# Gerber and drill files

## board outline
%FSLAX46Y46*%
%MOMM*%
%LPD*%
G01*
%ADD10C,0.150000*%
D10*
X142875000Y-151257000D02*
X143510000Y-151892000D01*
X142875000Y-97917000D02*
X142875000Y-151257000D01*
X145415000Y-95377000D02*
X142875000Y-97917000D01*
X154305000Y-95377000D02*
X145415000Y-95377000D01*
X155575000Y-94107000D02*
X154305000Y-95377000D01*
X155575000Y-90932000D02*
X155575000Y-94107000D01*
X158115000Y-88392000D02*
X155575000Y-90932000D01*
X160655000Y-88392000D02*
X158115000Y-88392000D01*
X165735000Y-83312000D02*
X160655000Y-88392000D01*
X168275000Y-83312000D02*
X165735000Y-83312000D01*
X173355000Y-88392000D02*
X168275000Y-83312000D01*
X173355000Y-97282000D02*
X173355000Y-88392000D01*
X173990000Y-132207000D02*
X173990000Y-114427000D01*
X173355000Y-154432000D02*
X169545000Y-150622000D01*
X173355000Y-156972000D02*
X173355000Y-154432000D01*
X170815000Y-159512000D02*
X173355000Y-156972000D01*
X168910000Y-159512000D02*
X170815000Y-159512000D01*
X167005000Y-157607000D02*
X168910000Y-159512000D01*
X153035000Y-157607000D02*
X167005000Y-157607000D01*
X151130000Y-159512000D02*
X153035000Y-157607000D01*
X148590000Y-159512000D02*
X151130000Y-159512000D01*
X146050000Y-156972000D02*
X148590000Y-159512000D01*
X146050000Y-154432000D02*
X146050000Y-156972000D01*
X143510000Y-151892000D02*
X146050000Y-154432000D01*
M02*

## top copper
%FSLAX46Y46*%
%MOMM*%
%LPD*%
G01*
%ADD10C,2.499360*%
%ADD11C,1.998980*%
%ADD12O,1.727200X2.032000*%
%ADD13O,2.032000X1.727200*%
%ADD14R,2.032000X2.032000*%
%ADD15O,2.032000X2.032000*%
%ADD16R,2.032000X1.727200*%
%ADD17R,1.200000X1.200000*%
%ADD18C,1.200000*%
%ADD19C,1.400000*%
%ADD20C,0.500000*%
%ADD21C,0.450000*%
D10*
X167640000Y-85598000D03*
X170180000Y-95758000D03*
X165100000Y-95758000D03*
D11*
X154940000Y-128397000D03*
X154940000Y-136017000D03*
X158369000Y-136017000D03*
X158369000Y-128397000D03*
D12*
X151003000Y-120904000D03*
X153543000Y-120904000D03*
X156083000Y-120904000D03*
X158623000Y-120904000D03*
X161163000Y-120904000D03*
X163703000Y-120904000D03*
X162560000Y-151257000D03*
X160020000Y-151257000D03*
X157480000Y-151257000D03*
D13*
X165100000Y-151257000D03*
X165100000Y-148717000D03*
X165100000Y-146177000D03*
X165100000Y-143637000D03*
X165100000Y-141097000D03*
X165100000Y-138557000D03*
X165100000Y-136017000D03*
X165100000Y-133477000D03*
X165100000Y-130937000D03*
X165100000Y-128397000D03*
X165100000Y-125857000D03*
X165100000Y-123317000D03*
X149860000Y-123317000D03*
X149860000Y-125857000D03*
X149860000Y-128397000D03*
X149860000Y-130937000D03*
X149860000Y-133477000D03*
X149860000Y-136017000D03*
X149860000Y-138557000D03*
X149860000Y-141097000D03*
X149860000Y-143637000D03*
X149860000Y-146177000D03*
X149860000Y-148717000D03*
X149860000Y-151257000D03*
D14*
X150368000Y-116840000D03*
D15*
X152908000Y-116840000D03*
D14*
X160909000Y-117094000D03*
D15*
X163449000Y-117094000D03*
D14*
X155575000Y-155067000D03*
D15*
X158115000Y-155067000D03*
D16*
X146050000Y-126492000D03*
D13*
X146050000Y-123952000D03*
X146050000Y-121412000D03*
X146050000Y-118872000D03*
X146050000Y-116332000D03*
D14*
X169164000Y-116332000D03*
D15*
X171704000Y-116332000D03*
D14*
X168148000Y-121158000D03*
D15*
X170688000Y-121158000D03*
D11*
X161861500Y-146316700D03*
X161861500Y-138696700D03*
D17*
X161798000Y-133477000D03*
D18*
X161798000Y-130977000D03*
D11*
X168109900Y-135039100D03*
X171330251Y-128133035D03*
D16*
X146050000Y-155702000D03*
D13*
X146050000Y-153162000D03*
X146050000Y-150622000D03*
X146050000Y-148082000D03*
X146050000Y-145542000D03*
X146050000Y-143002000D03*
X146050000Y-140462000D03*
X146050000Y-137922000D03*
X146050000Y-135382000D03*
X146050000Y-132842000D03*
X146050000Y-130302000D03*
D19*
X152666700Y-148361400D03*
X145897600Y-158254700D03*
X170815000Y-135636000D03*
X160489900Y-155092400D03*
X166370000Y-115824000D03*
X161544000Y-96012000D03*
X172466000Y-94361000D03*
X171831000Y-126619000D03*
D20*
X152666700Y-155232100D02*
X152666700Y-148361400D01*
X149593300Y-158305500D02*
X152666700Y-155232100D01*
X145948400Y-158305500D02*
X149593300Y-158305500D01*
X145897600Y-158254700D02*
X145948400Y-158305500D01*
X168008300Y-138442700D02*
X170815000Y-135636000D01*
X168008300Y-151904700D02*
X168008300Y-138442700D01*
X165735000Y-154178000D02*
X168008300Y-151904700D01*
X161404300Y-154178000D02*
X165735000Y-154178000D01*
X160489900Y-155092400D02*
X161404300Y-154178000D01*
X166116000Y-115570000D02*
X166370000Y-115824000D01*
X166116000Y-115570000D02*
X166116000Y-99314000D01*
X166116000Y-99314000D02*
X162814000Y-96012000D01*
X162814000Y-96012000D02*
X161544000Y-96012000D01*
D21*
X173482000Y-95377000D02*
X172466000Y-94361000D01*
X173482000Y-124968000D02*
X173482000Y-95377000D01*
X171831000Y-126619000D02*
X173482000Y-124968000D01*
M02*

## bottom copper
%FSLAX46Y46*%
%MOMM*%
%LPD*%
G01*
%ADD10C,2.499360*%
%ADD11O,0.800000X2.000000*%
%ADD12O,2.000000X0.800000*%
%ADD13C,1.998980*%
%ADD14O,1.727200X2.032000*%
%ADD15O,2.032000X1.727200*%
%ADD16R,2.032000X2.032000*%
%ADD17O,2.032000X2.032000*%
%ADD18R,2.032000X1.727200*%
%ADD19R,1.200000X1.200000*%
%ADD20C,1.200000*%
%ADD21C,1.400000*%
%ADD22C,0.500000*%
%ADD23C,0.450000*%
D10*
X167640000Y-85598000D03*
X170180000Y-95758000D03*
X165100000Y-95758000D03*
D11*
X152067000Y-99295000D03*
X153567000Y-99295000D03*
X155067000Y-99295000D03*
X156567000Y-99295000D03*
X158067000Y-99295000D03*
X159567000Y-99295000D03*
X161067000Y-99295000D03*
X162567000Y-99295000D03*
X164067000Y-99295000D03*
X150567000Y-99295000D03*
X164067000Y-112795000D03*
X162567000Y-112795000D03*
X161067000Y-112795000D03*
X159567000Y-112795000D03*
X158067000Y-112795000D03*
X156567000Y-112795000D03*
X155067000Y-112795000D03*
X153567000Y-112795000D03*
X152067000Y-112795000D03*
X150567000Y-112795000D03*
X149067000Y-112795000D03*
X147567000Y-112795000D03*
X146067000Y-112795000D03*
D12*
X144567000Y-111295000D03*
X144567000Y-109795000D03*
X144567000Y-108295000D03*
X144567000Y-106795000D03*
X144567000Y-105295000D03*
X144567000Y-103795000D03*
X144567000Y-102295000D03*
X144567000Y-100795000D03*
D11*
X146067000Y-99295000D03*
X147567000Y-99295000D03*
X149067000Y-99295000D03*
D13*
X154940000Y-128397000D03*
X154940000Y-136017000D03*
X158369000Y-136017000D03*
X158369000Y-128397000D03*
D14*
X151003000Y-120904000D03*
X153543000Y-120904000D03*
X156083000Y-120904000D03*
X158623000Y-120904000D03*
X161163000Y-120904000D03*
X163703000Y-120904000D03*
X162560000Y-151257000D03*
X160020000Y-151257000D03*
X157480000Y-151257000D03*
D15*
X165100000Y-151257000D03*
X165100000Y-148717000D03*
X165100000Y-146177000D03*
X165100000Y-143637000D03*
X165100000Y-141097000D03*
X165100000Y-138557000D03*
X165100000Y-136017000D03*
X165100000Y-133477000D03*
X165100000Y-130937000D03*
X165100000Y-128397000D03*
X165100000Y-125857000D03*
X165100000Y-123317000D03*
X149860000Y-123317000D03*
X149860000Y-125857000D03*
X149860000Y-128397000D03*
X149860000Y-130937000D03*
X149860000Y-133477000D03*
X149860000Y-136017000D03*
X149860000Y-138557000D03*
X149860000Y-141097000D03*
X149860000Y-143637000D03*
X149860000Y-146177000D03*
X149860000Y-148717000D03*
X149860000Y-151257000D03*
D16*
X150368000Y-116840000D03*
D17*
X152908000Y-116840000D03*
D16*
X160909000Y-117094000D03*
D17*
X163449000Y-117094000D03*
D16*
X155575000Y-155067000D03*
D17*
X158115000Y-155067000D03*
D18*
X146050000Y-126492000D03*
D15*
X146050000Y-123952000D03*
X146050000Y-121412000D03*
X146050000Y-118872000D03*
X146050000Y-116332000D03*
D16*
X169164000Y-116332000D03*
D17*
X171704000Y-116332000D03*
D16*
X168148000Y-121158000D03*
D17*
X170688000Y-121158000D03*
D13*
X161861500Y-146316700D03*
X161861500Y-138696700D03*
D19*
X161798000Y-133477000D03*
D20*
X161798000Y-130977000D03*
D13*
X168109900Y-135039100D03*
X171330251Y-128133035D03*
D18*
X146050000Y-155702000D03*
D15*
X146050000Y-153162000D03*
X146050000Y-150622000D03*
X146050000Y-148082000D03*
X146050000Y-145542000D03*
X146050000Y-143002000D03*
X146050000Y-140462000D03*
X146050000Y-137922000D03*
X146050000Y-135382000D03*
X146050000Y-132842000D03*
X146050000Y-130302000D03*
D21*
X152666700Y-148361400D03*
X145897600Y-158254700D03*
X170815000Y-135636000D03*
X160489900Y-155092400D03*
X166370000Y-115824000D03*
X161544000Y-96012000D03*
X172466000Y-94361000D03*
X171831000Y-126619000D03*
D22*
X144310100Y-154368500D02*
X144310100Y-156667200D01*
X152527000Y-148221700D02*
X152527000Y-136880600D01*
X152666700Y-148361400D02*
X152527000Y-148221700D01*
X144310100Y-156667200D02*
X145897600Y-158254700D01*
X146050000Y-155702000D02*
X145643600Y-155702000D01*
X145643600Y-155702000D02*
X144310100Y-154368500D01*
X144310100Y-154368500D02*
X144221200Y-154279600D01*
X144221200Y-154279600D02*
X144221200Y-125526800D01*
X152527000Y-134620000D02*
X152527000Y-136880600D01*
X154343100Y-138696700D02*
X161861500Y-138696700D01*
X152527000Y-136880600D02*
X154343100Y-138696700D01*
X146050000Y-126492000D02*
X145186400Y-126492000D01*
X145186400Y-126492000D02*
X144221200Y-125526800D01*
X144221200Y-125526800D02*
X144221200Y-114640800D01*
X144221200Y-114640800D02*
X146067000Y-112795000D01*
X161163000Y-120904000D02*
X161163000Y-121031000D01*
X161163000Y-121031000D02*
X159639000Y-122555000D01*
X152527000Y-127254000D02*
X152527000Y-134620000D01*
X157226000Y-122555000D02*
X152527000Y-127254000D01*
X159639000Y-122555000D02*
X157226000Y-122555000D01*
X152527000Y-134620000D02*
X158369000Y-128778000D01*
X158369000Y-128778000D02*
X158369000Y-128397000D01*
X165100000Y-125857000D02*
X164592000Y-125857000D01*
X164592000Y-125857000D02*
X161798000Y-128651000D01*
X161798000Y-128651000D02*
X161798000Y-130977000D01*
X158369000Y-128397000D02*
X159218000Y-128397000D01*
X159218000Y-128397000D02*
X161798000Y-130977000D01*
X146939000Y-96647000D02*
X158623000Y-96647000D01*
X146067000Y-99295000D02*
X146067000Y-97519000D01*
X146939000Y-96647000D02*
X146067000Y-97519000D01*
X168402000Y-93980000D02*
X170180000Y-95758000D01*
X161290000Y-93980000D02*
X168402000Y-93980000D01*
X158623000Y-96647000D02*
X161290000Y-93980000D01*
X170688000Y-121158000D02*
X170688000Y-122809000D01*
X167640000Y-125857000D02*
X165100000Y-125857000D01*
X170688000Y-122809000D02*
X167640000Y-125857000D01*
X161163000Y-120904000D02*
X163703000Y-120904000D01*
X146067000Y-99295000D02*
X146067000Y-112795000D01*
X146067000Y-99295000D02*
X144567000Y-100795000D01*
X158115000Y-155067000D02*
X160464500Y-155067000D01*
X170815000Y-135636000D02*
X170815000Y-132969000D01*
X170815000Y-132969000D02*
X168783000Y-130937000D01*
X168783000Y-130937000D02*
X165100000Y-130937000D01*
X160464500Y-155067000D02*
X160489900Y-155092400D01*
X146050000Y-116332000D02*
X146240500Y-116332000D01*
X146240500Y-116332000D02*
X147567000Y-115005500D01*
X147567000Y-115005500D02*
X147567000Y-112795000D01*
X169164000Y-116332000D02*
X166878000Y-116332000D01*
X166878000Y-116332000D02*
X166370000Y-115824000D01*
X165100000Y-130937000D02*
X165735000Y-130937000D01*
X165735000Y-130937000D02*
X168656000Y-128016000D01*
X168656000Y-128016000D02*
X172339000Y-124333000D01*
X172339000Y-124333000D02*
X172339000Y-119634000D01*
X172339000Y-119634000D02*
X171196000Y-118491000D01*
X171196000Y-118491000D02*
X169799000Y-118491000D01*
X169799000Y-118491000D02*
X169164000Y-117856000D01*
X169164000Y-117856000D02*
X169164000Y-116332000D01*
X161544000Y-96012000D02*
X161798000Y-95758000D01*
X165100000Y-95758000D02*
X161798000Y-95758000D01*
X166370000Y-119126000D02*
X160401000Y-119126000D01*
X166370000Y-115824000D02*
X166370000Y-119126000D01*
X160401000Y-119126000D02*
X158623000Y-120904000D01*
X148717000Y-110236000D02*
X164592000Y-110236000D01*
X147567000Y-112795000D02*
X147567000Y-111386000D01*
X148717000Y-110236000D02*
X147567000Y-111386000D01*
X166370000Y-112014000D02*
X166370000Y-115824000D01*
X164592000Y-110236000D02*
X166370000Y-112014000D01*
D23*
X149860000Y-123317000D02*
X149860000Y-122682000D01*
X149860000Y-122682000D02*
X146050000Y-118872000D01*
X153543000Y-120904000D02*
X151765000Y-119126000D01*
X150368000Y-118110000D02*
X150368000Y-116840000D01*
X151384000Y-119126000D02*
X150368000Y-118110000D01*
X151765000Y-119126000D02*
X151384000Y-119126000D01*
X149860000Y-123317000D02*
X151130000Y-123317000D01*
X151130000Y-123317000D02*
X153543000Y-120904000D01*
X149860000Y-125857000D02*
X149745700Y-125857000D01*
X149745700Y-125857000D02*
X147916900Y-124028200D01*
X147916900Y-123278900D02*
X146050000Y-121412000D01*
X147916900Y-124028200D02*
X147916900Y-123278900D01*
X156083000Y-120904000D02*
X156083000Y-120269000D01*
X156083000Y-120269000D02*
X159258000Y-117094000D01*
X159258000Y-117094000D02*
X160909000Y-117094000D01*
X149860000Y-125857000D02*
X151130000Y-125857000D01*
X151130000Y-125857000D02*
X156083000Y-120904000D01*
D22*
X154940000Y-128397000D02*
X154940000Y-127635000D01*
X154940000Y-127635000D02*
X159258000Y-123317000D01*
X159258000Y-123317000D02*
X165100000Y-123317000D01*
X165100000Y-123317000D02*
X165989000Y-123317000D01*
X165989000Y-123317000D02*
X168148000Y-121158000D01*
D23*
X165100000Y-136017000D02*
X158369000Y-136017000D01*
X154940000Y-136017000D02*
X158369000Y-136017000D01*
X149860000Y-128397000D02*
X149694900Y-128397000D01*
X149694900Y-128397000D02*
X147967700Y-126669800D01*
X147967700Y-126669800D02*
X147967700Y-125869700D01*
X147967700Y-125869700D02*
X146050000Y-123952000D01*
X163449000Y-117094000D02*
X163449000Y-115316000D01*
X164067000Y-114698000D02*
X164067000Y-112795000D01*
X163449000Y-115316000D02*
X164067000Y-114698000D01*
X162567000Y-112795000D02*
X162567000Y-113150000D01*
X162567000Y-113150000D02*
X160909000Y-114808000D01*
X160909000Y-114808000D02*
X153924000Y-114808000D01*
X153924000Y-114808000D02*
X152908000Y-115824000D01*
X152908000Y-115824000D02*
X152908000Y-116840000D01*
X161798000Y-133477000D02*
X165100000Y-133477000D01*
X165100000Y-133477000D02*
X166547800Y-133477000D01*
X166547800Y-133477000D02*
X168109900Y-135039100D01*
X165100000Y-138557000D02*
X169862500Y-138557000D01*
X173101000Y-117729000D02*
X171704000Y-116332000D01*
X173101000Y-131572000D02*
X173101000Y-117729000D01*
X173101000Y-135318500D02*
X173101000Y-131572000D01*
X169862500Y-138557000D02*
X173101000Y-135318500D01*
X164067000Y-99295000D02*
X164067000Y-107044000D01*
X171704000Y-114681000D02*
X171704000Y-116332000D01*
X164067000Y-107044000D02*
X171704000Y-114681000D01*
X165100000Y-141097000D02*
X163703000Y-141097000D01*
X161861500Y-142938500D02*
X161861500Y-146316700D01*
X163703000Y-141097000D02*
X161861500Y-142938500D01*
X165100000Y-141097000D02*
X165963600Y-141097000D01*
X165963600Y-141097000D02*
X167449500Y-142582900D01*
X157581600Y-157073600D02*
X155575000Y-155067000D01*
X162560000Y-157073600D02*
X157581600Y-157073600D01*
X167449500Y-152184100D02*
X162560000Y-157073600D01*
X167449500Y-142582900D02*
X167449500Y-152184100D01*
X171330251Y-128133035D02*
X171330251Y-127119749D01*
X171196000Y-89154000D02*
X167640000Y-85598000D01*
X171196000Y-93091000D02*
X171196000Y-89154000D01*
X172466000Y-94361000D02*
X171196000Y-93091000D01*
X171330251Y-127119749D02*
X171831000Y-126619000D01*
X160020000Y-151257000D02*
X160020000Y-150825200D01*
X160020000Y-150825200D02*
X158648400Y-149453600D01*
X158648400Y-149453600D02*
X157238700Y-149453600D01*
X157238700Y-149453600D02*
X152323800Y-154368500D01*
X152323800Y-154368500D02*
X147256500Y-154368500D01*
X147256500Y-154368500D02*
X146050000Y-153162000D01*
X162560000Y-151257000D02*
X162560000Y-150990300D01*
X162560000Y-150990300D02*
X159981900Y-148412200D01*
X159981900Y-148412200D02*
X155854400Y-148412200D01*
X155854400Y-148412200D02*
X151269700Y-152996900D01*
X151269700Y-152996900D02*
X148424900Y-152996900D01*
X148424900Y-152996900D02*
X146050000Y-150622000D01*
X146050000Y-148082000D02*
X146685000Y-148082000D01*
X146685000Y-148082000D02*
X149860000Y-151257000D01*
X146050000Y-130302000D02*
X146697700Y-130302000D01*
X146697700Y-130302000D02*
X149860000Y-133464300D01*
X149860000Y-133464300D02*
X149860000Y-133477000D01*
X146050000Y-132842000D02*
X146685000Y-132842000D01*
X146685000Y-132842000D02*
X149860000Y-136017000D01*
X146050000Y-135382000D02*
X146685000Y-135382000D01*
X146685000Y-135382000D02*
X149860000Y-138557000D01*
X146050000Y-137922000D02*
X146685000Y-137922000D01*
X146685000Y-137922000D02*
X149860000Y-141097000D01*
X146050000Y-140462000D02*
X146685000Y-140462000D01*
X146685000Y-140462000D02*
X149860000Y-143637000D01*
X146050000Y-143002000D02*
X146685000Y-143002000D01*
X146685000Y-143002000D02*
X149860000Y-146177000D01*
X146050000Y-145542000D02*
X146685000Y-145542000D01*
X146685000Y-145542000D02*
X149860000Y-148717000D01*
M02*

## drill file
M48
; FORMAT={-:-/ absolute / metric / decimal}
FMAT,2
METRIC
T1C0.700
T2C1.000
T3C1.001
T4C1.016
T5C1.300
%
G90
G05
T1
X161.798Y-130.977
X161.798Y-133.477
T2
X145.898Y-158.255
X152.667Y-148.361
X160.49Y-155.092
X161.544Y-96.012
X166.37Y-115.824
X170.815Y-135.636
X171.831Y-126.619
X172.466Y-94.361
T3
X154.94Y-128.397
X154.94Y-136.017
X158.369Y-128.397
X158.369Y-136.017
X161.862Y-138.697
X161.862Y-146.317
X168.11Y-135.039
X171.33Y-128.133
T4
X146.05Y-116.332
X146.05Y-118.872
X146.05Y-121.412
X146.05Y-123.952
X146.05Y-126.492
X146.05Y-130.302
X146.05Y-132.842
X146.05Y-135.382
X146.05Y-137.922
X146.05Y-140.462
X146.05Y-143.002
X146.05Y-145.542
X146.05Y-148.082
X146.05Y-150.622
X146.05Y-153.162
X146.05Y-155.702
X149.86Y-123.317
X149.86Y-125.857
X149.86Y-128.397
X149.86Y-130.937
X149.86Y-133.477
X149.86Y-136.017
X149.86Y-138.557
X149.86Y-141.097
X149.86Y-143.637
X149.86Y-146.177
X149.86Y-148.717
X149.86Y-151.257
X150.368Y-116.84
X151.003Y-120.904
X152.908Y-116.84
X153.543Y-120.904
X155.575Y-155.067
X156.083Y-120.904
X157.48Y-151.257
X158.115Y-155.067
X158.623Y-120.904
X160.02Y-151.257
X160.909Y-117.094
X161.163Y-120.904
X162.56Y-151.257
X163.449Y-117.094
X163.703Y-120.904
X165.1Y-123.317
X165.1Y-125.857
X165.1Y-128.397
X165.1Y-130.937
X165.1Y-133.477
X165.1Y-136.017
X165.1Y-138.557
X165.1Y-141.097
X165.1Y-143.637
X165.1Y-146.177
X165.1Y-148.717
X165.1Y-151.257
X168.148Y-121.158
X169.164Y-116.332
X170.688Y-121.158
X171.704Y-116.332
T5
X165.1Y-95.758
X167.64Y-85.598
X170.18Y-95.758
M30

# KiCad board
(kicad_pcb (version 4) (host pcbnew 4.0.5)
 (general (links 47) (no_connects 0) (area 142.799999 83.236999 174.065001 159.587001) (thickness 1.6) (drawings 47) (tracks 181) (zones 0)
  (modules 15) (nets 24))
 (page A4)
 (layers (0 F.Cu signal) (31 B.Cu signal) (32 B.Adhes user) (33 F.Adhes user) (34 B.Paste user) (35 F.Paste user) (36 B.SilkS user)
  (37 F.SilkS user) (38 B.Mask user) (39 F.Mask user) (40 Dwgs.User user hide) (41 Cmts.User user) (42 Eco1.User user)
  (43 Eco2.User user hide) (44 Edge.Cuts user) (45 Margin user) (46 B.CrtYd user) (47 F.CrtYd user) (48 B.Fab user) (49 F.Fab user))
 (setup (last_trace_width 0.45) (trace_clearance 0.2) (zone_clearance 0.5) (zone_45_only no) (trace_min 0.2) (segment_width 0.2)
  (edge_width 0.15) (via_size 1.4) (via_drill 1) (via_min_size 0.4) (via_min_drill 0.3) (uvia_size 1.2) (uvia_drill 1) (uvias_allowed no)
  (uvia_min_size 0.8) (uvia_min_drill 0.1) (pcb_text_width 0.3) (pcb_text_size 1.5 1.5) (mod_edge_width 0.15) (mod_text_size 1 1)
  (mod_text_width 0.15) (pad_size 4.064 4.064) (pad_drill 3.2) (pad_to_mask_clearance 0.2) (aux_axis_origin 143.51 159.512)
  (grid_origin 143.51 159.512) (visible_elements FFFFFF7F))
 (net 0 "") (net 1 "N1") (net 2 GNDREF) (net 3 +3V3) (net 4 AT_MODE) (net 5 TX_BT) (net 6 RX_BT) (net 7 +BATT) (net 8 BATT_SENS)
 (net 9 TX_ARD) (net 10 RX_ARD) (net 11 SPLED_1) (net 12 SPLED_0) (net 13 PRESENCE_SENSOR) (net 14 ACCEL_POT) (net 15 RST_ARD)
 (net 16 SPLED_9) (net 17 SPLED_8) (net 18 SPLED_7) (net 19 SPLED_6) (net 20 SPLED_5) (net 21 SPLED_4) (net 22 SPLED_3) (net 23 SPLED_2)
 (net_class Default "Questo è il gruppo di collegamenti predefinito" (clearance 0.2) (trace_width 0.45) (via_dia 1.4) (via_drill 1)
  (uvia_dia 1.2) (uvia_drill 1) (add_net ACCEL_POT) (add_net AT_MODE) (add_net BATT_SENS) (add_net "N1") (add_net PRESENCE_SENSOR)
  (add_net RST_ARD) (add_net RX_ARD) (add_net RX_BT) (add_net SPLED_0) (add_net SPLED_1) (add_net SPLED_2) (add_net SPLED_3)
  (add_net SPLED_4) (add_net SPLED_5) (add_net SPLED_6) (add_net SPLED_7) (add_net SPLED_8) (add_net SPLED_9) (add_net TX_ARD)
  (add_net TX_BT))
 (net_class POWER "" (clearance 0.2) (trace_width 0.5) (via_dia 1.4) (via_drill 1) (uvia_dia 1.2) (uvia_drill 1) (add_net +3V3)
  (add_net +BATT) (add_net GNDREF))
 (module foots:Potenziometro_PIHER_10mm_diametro (layer F.Cu) (at 165.1 95.758)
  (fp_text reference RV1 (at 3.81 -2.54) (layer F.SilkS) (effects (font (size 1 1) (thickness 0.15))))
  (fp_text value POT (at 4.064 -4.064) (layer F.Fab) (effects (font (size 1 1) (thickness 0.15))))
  (pad 2 thru_hole circle (at 2.54 -10.16) (size 2.49936 2.49936) (drill 1.30048) (layers *.Cu *.Mask) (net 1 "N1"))
  (pad 3 thru_hole circle (at 5.08 0) (size 2.49936 2.49936) (drill 1.30048) (layers *.Cu *.Mask) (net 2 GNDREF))
  (pad 1 thru_hole circle (at 0 0) (size 2.49936 2.49936) (drill 1.30048) (layers *.Cu *.Mask) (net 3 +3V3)))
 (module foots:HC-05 (layer B.Cu) (at 155.067 106.045 90)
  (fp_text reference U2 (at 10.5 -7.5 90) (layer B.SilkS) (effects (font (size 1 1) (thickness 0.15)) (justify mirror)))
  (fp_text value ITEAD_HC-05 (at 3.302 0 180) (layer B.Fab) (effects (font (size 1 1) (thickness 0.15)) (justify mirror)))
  (pad 26 smd oval (at 6.75 -3 90) (size 2 0.8) (layers B.Cu B.Paste B.Mask))
  (pad 27 smd oval (at 6.75 -1.5 90) (size 2 0.8) (layers B.Cu B.Paste B.Mask))
  (pad 28 smd oval (at 6.75 0 90) (size 2 0.8) (layers B.Cu B.Paste B.Mask))
  (pad 29 smd oval (at 6.75 1.5 90) (size 2 0.8) (layers B.Cu B.Paste B.Mask))
  (pad 30 smd oval (at 6.75 3 90) (size 2 0.8) (layers B.Cu B.Paste B.Mask))
  (pad 31 smd oval (at 6.75 4.5 90) (size 2 0.8) (layers B.Cu B.Paste B.Mask))
  (pad 32 smd oval (at 6.75 6 90) (size 2 0.8) (layers B.Cu B.Paste B.Mask))
  (pad 33 smd oval (at 6.75 7.5 90) (size 2 0.8) (layers B.Cu B.Paste B.Mask))
  (pad 34 smd oval (at 6.75 9 90) (size 2 0.8) (layers B.Cu B.Paste B.Mask) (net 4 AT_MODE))
  (pad 25 smd oval (at 6.75 -4.5 90) (size 2 0.8) (layers B.Cu B.Paste B.Mask))
  (pad 1 smd oval (at -6.75 9 90) (size 2 0.8) (layers B.Cu B.Paste B.Mask) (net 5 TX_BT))
  (pad 2 smd oval (at -6.75 7.5 90) (size 2 0.8) (layers B.Cu B.Paste B.Mask) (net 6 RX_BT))
  (pad 3 smd oval (at -6.75 6 90) (size 2 0.8) (layers B.Cu B.Paste B.Mask))
  (pad 4 smd oval (at -6.75 4.5 90) (size 2 0.8) (layers B.Cu B.Paste B.Mask))
  (pad 5 smd oval (at -6.75 3 90) (size 2 0.8) (layers B.Cu B.Paste B.Mask))
  (pad 6 smd oval (at -6.75 1.5 90) (size 2 0.8) (layers B.Cu B.Paste B.Mask))
  (pad 7 smd oval (at -6.75 0 90) (size 2 0.8) (layers B.Cu B.Paste B.Mask))
  (pad 8 smd oval (at -6.75 -1.5 90) (size 2 0.8) (layers B.Cu B.Paste B.Mask))
  (pad 9 smd oval (at -6.75 -3 90) (size 2 0.8) (layers B.Cu B.Paste B.Mask))
  (pad 10 smd oval (at -6.75 -4.5 90) (size 2 0.8) (layers B.Cu B.Paste B.Mask))
  (pad 11 smd oval (at -6.75 -6 90) (size 2 0.8) (layers B.Cu B.Paste B.Mask))
  (pad 12 smd oval (at -6.75 -7.5 90) (size 2 0.8) (layers B.Cu B.Paste B.Mask) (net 3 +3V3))
  (pad 13 smd oval (at -6.75 -9 90) (size 2 0.8) (layers B.Cu B.Paste B.Mask) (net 2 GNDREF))
  (pad 14 smd oval (at -5.25 -10.5) (size 2 0.8) (layers B.Cu B.Paste B.Mask))
  (pad 15 smd oval (at -3.75 -10.5 180) (size 2 0.8) (layers B.Cu B.Paste B.Mask))
  (pad 16 smd oval (at -2.25 -10.5 180) (size 2 0.8) (layers B.Cu B.Paste B.Mask))
  (pad 17 smd oval (at -0.75 -10.5 180) (size 2 0.8) (layers B.Cu B.Paste B.Mask))
  (pad 18 smd oval (at 0.75 -10.5 180) (size 2 0.8) (layers B.Cu B.Paste B.Mask))
  (pad 19 smd oval (at 2.25 -10.5 180) (size 2 0.8) (layers B.Cu B.Paste B.Mask))
  (pad 20 smd oval (at 3.75 -10.5 180) (size 2 0.8) (layers B.Cu B.Paste B.Mask))
  (pad 21 smd oval (at 5.25 -10.5 180) (size 2 0.8) (layers B.Cu B.Paste B.Mask) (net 2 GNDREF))
  (pad 22 smd oval (at 6.75 -9 90) (size 2 0.8) (layers B.Cu B.Paste B.Mask) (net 2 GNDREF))
  (pad 23 smd oval (at 6.75 -7.5 90) (size 2 0.8) (layers B.Cu B.Paste B.Mask))
  (pad 24 smd oval (at 6.75 -6 90) (size 2 0.8) (layers B.Cu B.Paste B.Mask)))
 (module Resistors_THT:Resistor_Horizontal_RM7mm (layer F.Cu) (at 154.94 128.397 270)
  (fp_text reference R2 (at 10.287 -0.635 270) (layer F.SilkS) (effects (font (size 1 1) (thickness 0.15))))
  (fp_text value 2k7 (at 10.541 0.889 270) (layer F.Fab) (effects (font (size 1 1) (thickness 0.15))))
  (pad 1 thru_hole circle (at 0 0 270) (size 1.99898 1.99898) (drill 1.00076) (layers *.Cu *.SilkS *.Mask) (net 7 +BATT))
  (pad 2 thru_hole circle (at 7.62 0 270) (size 1.99898 1.99898) (drill 1.00076) (layers *.Cu *.SilkS *.Mask) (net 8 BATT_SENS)))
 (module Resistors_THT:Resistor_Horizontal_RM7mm (layer F.Cu) (at 158.369 136.017 90)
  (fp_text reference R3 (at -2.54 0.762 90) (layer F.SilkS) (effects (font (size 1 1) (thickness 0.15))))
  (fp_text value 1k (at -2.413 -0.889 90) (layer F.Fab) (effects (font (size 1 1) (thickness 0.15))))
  (pad 1 thru_hole circle (at 0 0 90) (size 1.99898 1.99898) (drill 1.00076) (layers *.Cu *.SilkS *.Mask) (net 8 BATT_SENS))
  (pad 2 thru_hole circle (at 7.62 0 90) (size 1.99898 1.99898) (drill 1.00076) (layers *.Cu *.SilkS *.Mask)))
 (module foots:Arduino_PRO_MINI (layer F.Cu) (at 157.48 120.777)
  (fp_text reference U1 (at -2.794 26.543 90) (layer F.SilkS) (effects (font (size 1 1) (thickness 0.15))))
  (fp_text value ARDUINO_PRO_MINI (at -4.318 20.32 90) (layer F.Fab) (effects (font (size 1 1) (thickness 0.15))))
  (pad 33 thru_hole oval (at -6.477 0.127 90) (size 2.032 1.7272) (drill 1.016) (layers *.Cu *.Mask))
  (pad 32 thru_hole oval (at -3.937 0.127 90) (size 2.032 1.7272) (drill 1.016) (layers *.Cu *.Mask) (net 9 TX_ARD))
  (pad 31 thru_hole oval (at -1.397 0.127 90) (size 2.032 1.7272) (drill 1.016) (layers *.Cu *.Mask) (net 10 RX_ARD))
  (pad 30 thru_hole oval (at 1.143 0.127 90) (size 2.032 1.7272) (drill 1.016) (layers *.Cu *.Mask) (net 3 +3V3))
  (pad 29 thru_hole oval (at 3.683 0.127 90) (size 2.032 1.7272) (drill 1.016) (layers *.Cu *.Mask) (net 2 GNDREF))
  (pad 28 thru_hole oval (at 6.223 0.127 90) (size 2.032 1.7272) (drill 1.016) (layers *.Cu *.Mask) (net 2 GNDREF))
  (pad 15 thru_hole oval (at 5.08 30.48 90) (size 2.032 1.7272) (drill 1.016) (layers *.Cu *.Mask) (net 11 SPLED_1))
  (pad 14 thru_hole oval (at 2.54 30.48 90) (size 2.032 1.7272) (drill 1.016) (layers *.Cu *.Mask) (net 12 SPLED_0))
  (pad 13 thru_hole oval (at 0 30.48 90) (size 2.032 1.7272) (drill 1.016) (layers *.Cu *.Mask))
  (pad 16 thru_hole oval (at 7.62 30.48) (size 2.032 1.7272) (drill 1.016) (layers *.Cu *.Mask))
  (pad 17 thru_hole oval (at 7.62 27.94) (size 2.032 1.7272) (drill 1.016) (layers *.Cu *.Mask))
  (pad 18 thru_hole oval (at 7.62 25.4) (size 2.032 1.7272) (drill 1.016) (layers *.Cu *.Mask))
  (pad 19 thru_hole oval (at 7.62 22.86) (size 2.032 1.7272) (drill 1.016) (layers *.Cu *.Mask))
  (pad 20 thru_hole oval (at 7.62 20.32) (size 2.032 1.7272) (drill 1.016) (layers *.Cu *.Mask) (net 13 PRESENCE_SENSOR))
  (pad 21 thru_hole oval (at 7.62 17.78) (size 2.032 1.7272) (drill 1.016) (layers *.Cu *.Mask) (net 4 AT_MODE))
  (pad 22 thru_hole oval (at 7.62 15.24) (size 2.032 1.7272) (drill 1.016) (layers *.Cu *.Mask) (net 8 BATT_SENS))
  (pad 23 thru_hole oval (at 7.62 12.7) (size 2.032 1.7272) (drill 1.016) (layers *.Cu *.Mask) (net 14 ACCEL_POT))
  (pad 24 thru_hole oval (at 7.62 10.16) (size 2.032 1.7272) (drill 1.016) (layers *.Cu *.Mask) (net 3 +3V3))
  (pad 25 thru_hole oval (at 7.62 7.62) (size 2.032 1.7272) (drill 1.016) (layers *.Cu *.Mask))
  (pad 26 thru_hole oval (at 7.62 5.08) (size 2.032 1.7272) (drill 1.016) (layers *.Cu *.Mask) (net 2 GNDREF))
  (pad 27 thru_hole oval (at 7.62 2.54) (size 2.032 1.7272) (drill 1.016) (layers *.Cu *.Mask) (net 7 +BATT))
  (pad 1 thru_hole oval (at -7.62 2.54) (size 2.032 1.7272) (drill 1.016) (layers *.Cu *.Mask) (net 9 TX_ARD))
  (pad 2 thru_hole oval (at -7.62 5.08) (size 2.032 1.7272) (drill 1.016) (layers *.Cu *.Mask) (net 10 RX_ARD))
  (pad 3 thru_hole oval (at -7.62 7.62) (size 2.032 1.7272) (drill 1.016) (layers *.Cu *.Mask) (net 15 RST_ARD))
  (pad 4 thru_hole oval (at -7.62 10.16) (size 2.032 1.7272) (drill 1.016) (layers *.Cu *.Mask))
  (pad 5 thru_hole oval (at -7.62 12.7) (size 2.032 1.7272) (drill 1.016) (layers *.Cu *.Mask) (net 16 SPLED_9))
  (pad 6 thru_hole oval (at -7.62 15.24) (size 2.032 1.7272) (drill 1.016) (layers *.Cu *.Mask) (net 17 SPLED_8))
  (pad 7 thru_hole oval (at -7.62 17.78) (size 2.032 1.7272) (drill 1.016) (layers *.Cu *.Mask) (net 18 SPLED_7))
  (pad 8 thru_hole oval (at -7.62 20.32) (size 2.032 1.7272) (drill 1.016) (layers *.Cu *.Mask) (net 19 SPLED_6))
  (pad 9 thru_hole oval (at -7.62 22.86) (size 2.032 1.7272) (drill 1.016) (layers *.Cu *.Mask) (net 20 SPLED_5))
  (pad 10 thru_hole oval (at -7.62 25.4) (size 2.032 1.7272) (drill 1.016) (layers *.Cu *.Mask) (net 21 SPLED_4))
  (pad 11 thru_hole oval (at -7.62 27.94) (size 2.032 1.7272) (drill 1.016) (layers *.Cu *.Mask) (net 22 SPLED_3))
  (pad 12 thru_hole oval (at -7.62 30.48) (size 2.032 1.7272) (drill 1.016) (layers *.Cu *.Mask) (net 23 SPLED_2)))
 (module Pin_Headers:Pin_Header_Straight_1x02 (layer F.Cu) (at 150.368 116.84 90)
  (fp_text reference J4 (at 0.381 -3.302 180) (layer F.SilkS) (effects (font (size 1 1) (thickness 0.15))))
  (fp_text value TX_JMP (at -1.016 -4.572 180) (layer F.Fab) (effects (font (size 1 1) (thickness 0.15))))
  (pad 1 thru_hole rect (at 0 0 90) (size 2.032 2.032) (drill 1.016) (layers *.Cu *.Mask) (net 9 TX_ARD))
  (pad 2 thru_hole oval (at 0 2.54 90) (size 2.032 2.032) (drill 1.016) (layers *.Cu *.Mask) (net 6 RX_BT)))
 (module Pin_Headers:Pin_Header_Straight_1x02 (layer F.Cu) (at 160.909 117.094 90)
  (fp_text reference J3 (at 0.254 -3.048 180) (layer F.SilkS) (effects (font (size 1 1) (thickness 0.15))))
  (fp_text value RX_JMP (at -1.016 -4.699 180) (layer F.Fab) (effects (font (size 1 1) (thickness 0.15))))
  (pad 1 thru_hole rect (at 0 0 90) (size 2.032 2.032) (drill 1.016) (layers *.Cu *.Mask) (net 10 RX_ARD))
  (pad 2 thru_hole oval (at 0 2.54 90) (size 2.032 2.032) (drill 1.016) (layers *.Cu *.Mask) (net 5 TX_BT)))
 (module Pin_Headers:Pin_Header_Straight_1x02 (layer F.Cu) (at 155.575 155.067 90)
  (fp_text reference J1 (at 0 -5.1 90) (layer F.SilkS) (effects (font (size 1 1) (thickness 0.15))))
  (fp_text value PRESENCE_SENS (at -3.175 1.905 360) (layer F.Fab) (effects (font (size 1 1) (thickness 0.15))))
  (pad 1 thru_hole rect (at 0 0 90) (size 2.032 2.032) (drill 1.016) (layers *.Cu *.Mask) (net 13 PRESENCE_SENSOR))
  (pad 2 thru_hole oval (at 0 2.54 90) (size 2.032 2.032) (drill 1.016) (layers *.Cu *.Mask) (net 3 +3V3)))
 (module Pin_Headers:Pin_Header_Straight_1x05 (layer F.Cu) (at 146.05 126.492 180)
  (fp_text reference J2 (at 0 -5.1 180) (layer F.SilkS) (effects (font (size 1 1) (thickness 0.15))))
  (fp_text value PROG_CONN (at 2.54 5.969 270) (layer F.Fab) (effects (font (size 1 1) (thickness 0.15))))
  (pad 1 thru_hole rect (at 0 0 180) (size 2.032 1.7272) (drill 1.016) (layers *.Cu *.Mask) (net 2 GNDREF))
  (pad 2 thru_hole oval (at 0 2.54 180) (size 2.032 1.7272) (drill 1.016) (layers *.Cu *.Mask) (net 15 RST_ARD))
  (pad 3 thru_hole oval (at 0 5.08 180) (size 2.032 1.7272) (drill 1.016) (layers *.Cu *.Mask) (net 10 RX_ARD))
  (pad 4 thru_hole oval (at 0 7.62 180) (size 2.032 1.7272) (drill 1.016) (layers *.Cu *.Mask) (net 9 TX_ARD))
  (pad 5 thru_hole oval (at 0 10.16 180) (size 2.032 1.7272) (drill 1.016) (layers *.Cu *.Mask) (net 3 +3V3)))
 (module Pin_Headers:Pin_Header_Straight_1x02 (layer F.Cu) (at 169.164 116.332 90)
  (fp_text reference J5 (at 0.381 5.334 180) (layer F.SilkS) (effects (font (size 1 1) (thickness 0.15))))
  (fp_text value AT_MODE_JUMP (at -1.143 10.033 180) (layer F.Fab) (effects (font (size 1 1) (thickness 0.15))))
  (pad 1 thru_hole rect (at 0 0 90) (size 2.032 2.032) (drill 1.016) (layers *.Cu *.Mask) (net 3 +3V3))
  (pad 2 thru_hole oval (at 0 2.54 90) (size 2.032 2.032) (drill 1.016) (layers *.Cu *.Mask) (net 4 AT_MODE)))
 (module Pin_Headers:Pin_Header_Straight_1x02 (layer F.Cu) (at 168.148 121.158 90)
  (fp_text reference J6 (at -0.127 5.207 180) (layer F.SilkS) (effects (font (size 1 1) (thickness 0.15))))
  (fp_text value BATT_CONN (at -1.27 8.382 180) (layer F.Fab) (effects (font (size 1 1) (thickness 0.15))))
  (pad 1 thru_hole rect (at 0 0 90) (size 2.032 2.032) (drill 1.016) (layers *.Cu *.Mask) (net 7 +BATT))
  (pad 2 thru_hole oval (at 0 2.54 90) (size 2.032 2.032) (drill 1.016) (layers *.Cu *.Mask) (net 2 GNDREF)))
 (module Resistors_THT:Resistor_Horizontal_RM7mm (layer F.Cu) (at 161.8615 146.3167 90)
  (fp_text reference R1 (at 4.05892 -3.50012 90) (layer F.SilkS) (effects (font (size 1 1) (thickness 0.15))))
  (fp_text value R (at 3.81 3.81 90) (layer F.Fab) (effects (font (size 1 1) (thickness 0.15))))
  (pad 1 thru_hole circle (at 0 0 90) (size 1.99898 1.99898) (drill 1.00076) (layers *.Cu *.SilkS *.Mask) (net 13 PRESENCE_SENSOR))
  (pad 2 thru_hole circle (at 7.62 0 90) (size 1.99898 1.99898) (drill 1.00076) (layers *.Cu *.SilkS *.Mask) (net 2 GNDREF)))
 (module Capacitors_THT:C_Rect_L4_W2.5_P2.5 (layer F.Cu) (at 161.798 133.477 90)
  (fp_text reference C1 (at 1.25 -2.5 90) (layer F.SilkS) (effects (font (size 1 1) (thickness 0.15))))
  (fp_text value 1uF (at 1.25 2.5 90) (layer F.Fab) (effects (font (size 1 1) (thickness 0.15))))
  (pad 1 thru_hole rect (at 0 0 90) (size 1.2 1.2) (drill 0.7) (layers *.Cu *.Mask) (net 14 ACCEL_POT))
  (pad 2 thru_hole circle (at 2.5 0 90) (size 1.2 1.2) (drill 0.7) (layers *.Cu *.Mask) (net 2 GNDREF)))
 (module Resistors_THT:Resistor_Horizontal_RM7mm (layer F.Cu) (at 168.1099 135.0391 65)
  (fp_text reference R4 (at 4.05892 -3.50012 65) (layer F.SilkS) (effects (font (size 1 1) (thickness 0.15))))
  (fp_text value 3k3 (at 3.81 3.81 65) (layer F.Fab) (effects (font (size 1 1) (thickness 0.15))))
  (pad 1 thru_hole circle (at 0 0 65) (size 1.99898 1.99898) (drill 1.00076) (layers *.Cu *.SilkS *.Mask) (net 14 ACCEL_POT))
  (pad 2 thru_hole circle (at 7.62 0 65) (size 1.99898 1.99898) (drill 1.00076) (layers *.Cu *.SilkS *.Mask) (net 1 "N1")))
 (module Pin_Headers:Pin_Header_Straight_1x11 (layer F.Cu) (at 146.05 155.702 180)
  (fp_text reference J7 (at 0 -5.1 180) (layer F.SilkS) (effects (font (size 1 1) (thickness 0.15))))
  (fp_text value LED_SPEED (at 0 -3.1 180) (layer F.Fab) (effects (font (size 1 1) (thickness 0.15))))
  (pad 1 thru_hole rect (at 0 0 180) (size 2.032 1.7272) (drill 1.016) (layers *.Cu *.Mask) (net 2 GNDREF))
  (pad 2 thru_hole oval (at 0 2.54 180) (size 2.032 1.7272) (drill 1.016) (layers *.Cu *.Mask) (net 12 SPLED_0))
  (pad 3 thru_hole oval (at 0 5.08 180) (size 2.032 1.7272) (drill 1.016) (layers *.Cu *.Mask) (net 11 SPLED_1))
  (pad 4 thru_hole oval (at 0 7.62 180) (size 2.032 1.7272) (drill 1.016) (layers *.Cu *.Mask) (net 23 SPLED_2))
  (pad 5 thru_hole oval (at 0 10.16 180) (size 2.032 1.7272) (drill 1.016) (layers *.Cu *.Mask) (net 22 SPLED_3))
  (pad 6 thru_hole oval (at 0 12.7 180) (size 2.032 1.7272) (drill 1.016) (layers *.Cu *.Mask) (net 21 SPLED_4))
  (pad 7 thru_hole oval (at 0 15.24 180) (size 2.032 1.7272) (drill 1.016) (layers *.Cu *.Mask) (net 20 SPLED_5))
  (pad 8 thru_hole oval (at 0 17.78 180) (size 2.032 1.7272) (drill 1.016) (layers *.Cu *.Mask) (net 19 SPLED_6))
  (pad 9 thru_hole oval (at 0 20.32 180) (size 2.032 1.7272) (drill 1.016) (layers *.Cu *.Mask) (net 18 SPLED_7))
  (pad 10 thru_hole oval (at 0 22.86 180) (size 2.032 1.7272) (drill 1.016) (layers *.Cu *.Mask) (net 17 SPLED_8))
  (pad 11 thru_hole oval (at 0 25.4 180) (size 2.032 1.7272) (drill 1.016) (layers *.Cu *.Mask) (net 16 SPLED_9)))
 (gr_line (start 142.875 151.257) (end 143.51 151.892) (angle 90) (layer Edge.Cuts) (width 0.15))
 (gr_line (start 142.875 97.917) (end 142.875 151.257) (angle 90) (layer Edge.Cuts) (width 0.15))
 (gr_line (start 145.415 95.377) (end 142.875 97.917) (angle 90) (layer Edge.Cuts) (width 0.15))
 (gr_line (start 154.305 95.377) (end 145.415 95.377) (angle 90) (layer Edge.Cuts) (width 0.15))
 (gr_line (start 155.575 94.107) (end 154.305 95.377) (angle 90) (layer Edge.Cuts) (width 0.15))
 (gr_line (start 155.575 90.932) (end 155.575 94.107) (angle 90) (layer Edge.Cuts) (width 0.15))
 (gr_line (start 158.115 88.392) (end 155.575 90.932) (angle 90) (layer Edge.Cuts) (width 0.15))
 (gr_line (start 160.655 88.392) (end 158.115 88.392) (angle 90) (layer Edge.Cuts) (width 0.15))
 (gr_line (start 165.735 83.312) (end 160.655 88.392) (angle 90) (layer Edge.Cuts) (width 0.15))
 (gr_line (start 168.275 83.312) (end 165.735 83.312) (angle 90) (layer Edge.Cuts) (width 0.15))
 (gr_line (start 173.355 88.392) (end 168.275 83.312) (angle 90) (layer Edge.Cuts) (width 0.15))
 (gr_line (start 173.355 97.282) (end 173.355 88.392) (angle 90) (layer Edge.Cuts) (width 0.15))
 (gr_line (start 173.99 132.207) (end 173.99 114.427) (angle 90) (layer Edge.Cuts) (width 0.15))
 (gr_line (start 173.355 154.432) (end 169.545 150.622) (angle 90) (layer Edge.Cuts) (width 0.15))
 (gr_line (start 173.355 156.972) (end 173.355 154.432) (angle 90) (layer Edge.Cuts) (width 0.15))
 (gr_line (start 170.815 159.512) (end 173.355 156.972) (angle 90) (layer Edge.Cuts) (width 0.15))
 (gr_line (start 168.91 159.512) (end 170.815 159.512) (angle 90) (layer Edge.Cuts) (width 0.15))
 (gr_line (start 167.005 157.607) (end 168.91 159.512) (angle 90) (layer Edge.Cuts) (width 0.15))
 (gr_line (start 153.035 157.607) (end 167.005 157.607) (angle 90) (layer Edge.Cuts) (width 0.15))
 (gr_line (start 151.13 159.512) (end 153.035 157.607) (angle 90) (layer Edge.Cuts) (width 0.15))
 (gr_line (start 148.59 159.512) (end 151.13 159.512) (angle 90) (layer Edge.Cuts) (width 0.15))
 (gr_line (start 146.05 156.972) (end 148.59 159.512) (angle 90) (layer Edge.Cuts) (width 0.15))
 (gr_line (start 146.05 154.432) (end 146.05 156.972) (angle 90) (layer Edge.Cuts) (width 0.15))
 (gr_line (start 143.51 151.892) (end 146.05 154.432) (angle 90) (layer Edge.Cuts) (width 0.15))
 (segment (start 144.3101 154.3685) (end 144.3101 156.6672) (width 0.5) (layer B.Cu) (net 2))
 (segment (start 152.527 148.2217) (end 152.527 136.8806) (width 0.5) (layer B.Cu) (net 2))
 (segment (start 152.6667 148.3614) (end 152.527 148.2217) (width 0.5) (layer B.Cu) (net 2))
 (via (at 152.6667 148.3614) (size 1.4) (drill 1) (layers F.Cu B.Cu) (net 2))
 (segment (start 152.6667 155.2321) (end 152.6667 148.3614) (width 0.5) (layer F.Cu) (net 2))
 (segment (start 149.5933 158.3055) (end 152.6667 155.2321) (width 0.5) (layer F.Cu) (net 2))
 (segment (start 145.9484 158.3055) (end 149.5933 158.3055) (width 0.5) (layer F.Cu) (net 2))
 (segment (start 145.8976 158.2547) (end 145.9484 158.3055) (width 0.5) (layer F.Cu) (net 2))
 (via (at 145.8976 158.2547) (size 1.4) (drill 1) (layers F.Cu B.Cu) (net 2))
 (segment (start 144.3101 156.6672) (end 145.8976 158.2547) (width 0.5) (layer B.Cu) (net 2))
 (segment (start 146.05 155.702) (end 145.6436 155.702) (width 0.5) (layer B.Cu) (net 2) (status C00000))
 (segment (start 145.6436 155.702) (end 144.3101 154.3685) (width 0.5) (layer B.Cu) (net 2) (status 400000))
 (segment (start 144.3101 154.3685) (end 144.2212 154.2796) (width 0.5) (layer B.Cu) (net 2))
 (segment (start 144.2212 154.2796) (end 144.2212 125.5268) (width 0.5) (layer B.Cu) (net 2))
 (segment (start 152.527 134.62) (end 152.527 136.8806) (width 0.5) (layer B.Cu) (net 2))
 (segment (start 154.3431 138.6967) (end 161.8615 138.6967) (width 0.5) (layer B.Cu) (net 2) (status 800000))
 (segment (start 152.527 136.8806) (end 154.3431 138.6967) (width 0.5) (layer B.Cu) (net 2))
 (segment (start 146.05 126.492) (end 145.1864 126.492) (width 0.5) (layer B.Cu) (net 2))
 (segment (start 145.1864 126.492) (end 144.2212 125.5268) (width 0.5) (layer B.Cu) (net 2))
 (segment (start 144.2212 125.5268) (end 144.2212 114.6408) (width 0.5) (layer B.Cu) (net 2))
 (segment (start 144.2212 114.6408) (end 146.067 112.795) (width 0.5) (layer B.Cu) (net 2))
 (segment (start 161.163 120.904) (end 161.163 121.031) (width 0.5) (layer B.Cu) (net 2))
 (segment (start 161.163 121.031) (end 159.639 122.555) (width 0.5) (layer B.Cu) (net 2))
 (segment (start 152.527 127.254) (end 152.527 134.62) (width 0.5) (layer B.Cu) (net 2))
 (segment (start 157.226 122.555) (end 152.527 127.254) (width 0.5) (layer B.Cu) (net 2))
 (segment (start 159.639 122.555) (end 157.226 122.555) (width 0.5) (layer B.Cu) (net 2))
 (segment (start 152.527 134.62) (end 158.369 128.778) (width 0.5) (layer B.Cu) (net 2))
 (segment (start 158.369 128.778) (end 158.369 128.397) (width 0.5) (layer B.Cu) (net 2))
 (segment (start 165.1 125.857) (end 164.592 125.857) (width 0.5) (layer B.Cu) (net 2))
 (segment (start 164.592 125.857) (end 161.798 128.651) (width 0.5) (layer B.Cu) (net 2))
 (segment (start 161.798 128.651) (end 161.798 130.977) (width 0.5) (layer B.Cu) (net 2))
 (segment (start 158.369 128.397) (end 159.218 128.397) (width 0.5) (layer B.Cu) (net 2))
 (segment (start 159.218 128.397) (end 161.798 130.977) (width 0.5) (layer B.Cu) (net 2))
 (segment (start 146.939 96.647) (end 158.623 96.647) (width 0.5) (layer B.Cu) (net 2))
 (segment (start 146.067 99.295) (end 146.067 97.519) (width 0.5) (layer B.Cu) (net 2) (status 10))
 (segment (start 146.939 96.647) (end 146.067 97.519) (width 0.5) (layer B.Cu) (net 2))
 (segment (start 168.402 93.98) (end 170.18 95.758) (width 0.5) (layer B.Cu) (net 2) (status 20))
 (segment (start 161.29 93.98) (end 168.402 93.98) (width 0.5) (layer B.Cu) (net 2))
 (segment (start 158.623 96.647) (end 161.29 93.98) (width 0.5) (layer B.Cu) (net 2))
 (segment (start 170.688 121.158) (end 170.688 122.809) (width 0.5) (layer B.Cu) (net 2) (status 10))
 (segment (start 167.64 125.857) (end 165.1 125.857) (width 0.5) (layer B.Cu) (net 2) (status 20))
 (segment (start 170.688 122.809) (end 167.64 125.857) (width 0.5) (layer B.Cu) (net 2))
 (segment (start 161.163 120.904) (end 163.703 120.904) (width 0.5) (layer B.Cu) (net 2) (status 30))
 (segment (start 146.067 99.295) (end 146.067 112.795) (width 0.5) (layer B.Cu) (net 2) (status 30))
 (segment (start 146.067 99.295) (end 144.567 100.795) (width 0.5) (layer B.Cu) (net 2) (status 30))
 (segment (start 158.115 155.067) (end 160.4645 155.067) (width 0.5) (layer B.Cu) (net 3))
 (via (at 170.815 135.636) (size 1.4) (drill 1) (layers F.Cu B.Cu) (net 3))
 (segment (start 170.815 135.636) (end 170.815 132.969) (width 0.5) (layer B.Cu) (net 3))
 (segment (start 170.815 132.969) (end 168.783 130.937) (width 0.5) (layer B.Cu) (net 3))
 (segment (start 168.783 130.937) (end 165.1 130.937) (width 0.5) (layer B.Cu) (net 3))
 (segment (start 168.0083 138.4427) (end 170.815 135.636) (width 0.5) (layer F.Cu) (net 3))
 (segment (start 168.0083 151.9047) (end 168.0083 138.4427) (width 0.5) (layer F.Cu) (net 3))
 (segment (start 165.735 154.178) (end 168.0083 151.9047) (width 0.5) (layer F.Cu) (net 3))
 (segment (start 161.4043 154.178) (end 165.735 154.178) (width 0.5) (layer F.Cu) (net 3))
 (segment (start 160.4899 155.0924) (end 161.4043 154.178) (width 0.5) (layer F.Cu) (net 3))
 (via (at 160.4899 155.0924) (size 1.4) (drill 1) (layers F.Cu B.Cu) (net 3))
 (segment (start 160.4645 155.067) (end 160.4899 155.0924) (width 0.5) (layer B.Cu) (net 3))
 (segment (start 146.05 116.332) (end 146.2405 116.332) (width 0.5) (layer B.Cu) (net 3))
 (segment (start 146.2405 116.332) (end 147.567 115.0055) (width 0.5) (layer B.Cu) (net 3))
 (segment (start 147.567 115.0055) (end 147.567 112.795) (width 0.5) (layer B.Cu) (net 3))
 (segment (start 169.164 116.332) (end 166.878 116.332) (width 0.5) (layer B.Cu) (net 3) (status 10))
 (segment (start 166.878 116.332) (end 166.37 115.824) (width 0.5) (layer B.Cu) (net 3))
 (segment (start 165.1 130.937) (end 165.735 130.937) (width 0.5) (layer B.Cu) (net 3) (status 30))
 (segment (start 165.735 130.937) (end 168.656 128.016) (width 0.5) (layer B.Cu) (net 3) (status 10))
 (segment (start 168.656 128.016) (end 172.339 124.333) (width 0.5) (layer B.Cu) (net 3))
 (segment (start 172.339 124.333) (end 172.339 119.634) (width 0.5) (layer B.Cu) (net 3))
 (segment (start 172.339 119.634) (end 171.196 118.491) (width 0.5) (layer B.Cu) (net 3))
 (segment (start 171.196 118.491) (end 169.799 118.491) (width 0.5) (layer B.Cu) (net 3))
 (segment (start 169.799 118.491) (end 169.164 117.856) (width 0.5) (layer B.Cu) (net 3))
 (segment (start 169.164 117.856) (end 169.164 116.332) (width 0.5) (layer B.Cu) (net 3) (status 20))
 (via (at 166.37 115.824) (size 1.4) (drill 1) (layers F.Cu B.Cu) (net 3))
 (segment (start 166.116 115.57) (end 166.37 115.824) (width 0.5) (layer F.Cu) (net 3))
 (segment (start 166.116 115.57) (end 166.116 99.314) (width 0.5) (layer F.Cu) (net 3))
 (segment (start 166.116 99.314) (end 162.814 96.012) (width 0.5) (layer F.Cu) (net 3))
 (segment (start 162.814 96.012) (end 161.544 96.012) (width 0.5) (layer F.Cu) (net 3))
 (via (at 161.544 96.012) (size 1.4) (drill 1) (layers F.Cu B.Cu) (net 3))
 (segment (start 161.544 96.012) (end 161.798 95.758) (width 0.5) (layer B.Cu) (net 3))
 (segment (start 165.1 95.758) (end 161.798 95.758) (width 0.5) (layer B.Cu) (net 3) (status 10))
 (segment (start 166.37 119.126) (end 160.401 119.126) (width 0.5) (layer B.Cu) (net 3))
 (segment (start 166.37 115.824) (end 166.37 119.126) (width 0.5) (layer B.Cu) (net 3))
 (segment (start 160.401 119.126) (end 158.623 120.904) (width 0.5) (layer B.Cu) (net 3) (status 20))
 (segment (start 148.717 110.236) (end 164.592 110.236) (width 0.5) (layer B.Cu) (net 3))
 (segment (start 147.567 112.795) (end 147.567 111.386) (width 0.5) (layer B.Cu) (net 3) (status 10))
 (segment (start 148.717 110.236) (end 147.567 111.386) (width 0.5) (layer B.Cu) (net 3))
 (segment (start 166.37 112.014) (end 166.37 115.824) (width 0.5) (layer B.Cu) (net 3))
 (segment (start 164.592 110.236) (end 166.37 112.014) (width 0.5) (layer B.Cu) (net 3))
 (segment (start 149.86 123.317) (end 149.86 122.682) (width 0.45) (layer B.Cu) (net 9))
 (segment (start 149.86 122.682) (end 146.05 118.872) (width 0.45) (layer B.Cu) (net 9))
 (segment (start 153.543 120.904) (end 151.765 119.126) (width 0.45) (layer B.Cu) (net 9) (status 10))
 (segment (start 150.368 118.11) (end 150.368 116.84) (width 0.45) (layer B.Cu) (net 9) (status 20))
 (segment (start 151.384 119.126) (end 150.368 118.11) (width 0.45) (layer B.Cu) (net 9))
 (segment (start 151.765 119.126) (end 151.384 119.126) (width 0.45) (layer B.Cu) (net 9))
 (segment (start 149.86 123.317) (end 151.13 123.317) (width 0.45) (layer B.Cu) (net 9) (status 10))
 (segment (start 151.13 123.317) (end 153.543 120.904) (width 0.45) (layer B.Cu) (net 9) (status 20))
 (segment (start 149.86 125.857) (end 149.7457 125.857) (width 0.45) (layer B.Cu) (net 10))
 (segment (start 149.7457 125.857) (end 147.9169 124.0282) (width 0.45) (layer B.Cu) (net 10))
 (segment (start 147.9169 123.2789) (end 146.05 121.412) (width 0.45) (layer B.Cu) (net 10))
 (segment (start 147.9169 124.0282) (end 147.9169 123.2789) (width 0.45) (layer B.Cu) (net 10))
 (segment (start 156.083 120.904) (end 156.083 120.269) (width 0.45) (layer B.Cu) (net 10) (status 30))
 (segment (start 156.083 120.269) (end 159.258 117.094) (width 0.45) (layer B.Cu) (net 10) (status 10))
 (segment (start 159.258 117.094) (end 160.909 117.094) (width 0.45) (layer B.Cu) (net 10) (status 20))
 (segment (start 149.86 125.857) (end 151.13 125.857) (width 0.45) (layer B.Cu) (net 10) (status 10))
 (segment (start 151.13 125.857) (end 156.083 120.904) (width 0.45) (layer B.Cu) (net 10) (status 20))
 (segment (start 154.94 128.397) (end 154.94 127.635) (width 0.5) (layer B.Cu) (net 7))
 (segment (start 154.94 127.635) (end 159.258 123.317) (width 0.5) (layer B.Cu) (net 7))
 (segment (start 159.258 123.317) (end 165.1 123.317) (width 0.5) (layer B.Cu) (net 7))
 (segment (start 165.1 123.317) (end 165.989 123.317) (width 0.5) (layer B.Cu) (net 7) (status 30))
 (segment (start 165.989 123.317) (end 168.148 121.158) (width 0.5) (layer B.Cu) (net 7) (status 30))
 (segment (start 165.1 136.017) (end 158.369 136.017) (width 0.45) (layer B.Cu) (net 8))
 (segment (start 154.94 136.017) (end 158.369 136.017) (width 0.45) (layer B.Cu) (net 8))
 (segment (start 149.86 128.397) (end 149.6949 128.397) (width 0.45) (layer B.Cu) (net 15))
 (segment (start 149.6949 128.397) (end 147.9677 126.6698) (width 0.45) (layer B.Cu) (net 15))
 (segment (start 147.9677 126.6698) (end 147.9677 125.8697) (width 0.45) (layer B.Cu) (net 15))
 (segment (start 147.9677 125.8697) (end 146.05 123.952) (width 0.45) (layer B.Cu) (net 15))
 (segment (start 163.449 117.094) (end 163.449 115.316) (width 0.45) (layer B.Cu) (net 5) (status 10))
 (segment (start 164.067 114.698) (end 164.067 112.795) (width 0.45) (layer B.Cu) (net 5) (status 20))
 (segment (start 163.449 115.316) (end 164.067 114.698) (width 0.45) (layer B.Cu) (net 5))
 (segment (start 162.567 112.795) (end 162.567 113.15) (width 0.45) (layer B.Cu) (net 6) (status 30))
 (segment (start 162.567 113.15) (end 160.909 114.808) (width 0.45) (layer B.Cu) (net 6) (status 10))
 (segment (start 160.909 114.808) (end 153.924 114.808) (width 0.45) (layer B.Cu) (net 6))
 (segment (start 153.924 114.808) (end 152.908 115.824) (width 0.45) (layer B.Cu) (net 6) (status 20))
 (segment (start 152.908 115.824) (end 152.908 116.84) (width 0.45) (layer B.Cu) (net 6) (status 30))
 (segment (start 161.798 133.477) (end 165.1 133.477) (width 0.45) (layer B.Cu) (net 14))
 (segment (start 165.1 133.477) (end 166.5478 133.477) (width 0.45) (layer B.Cu) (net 14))
 (segment (start 166.5478 133.477) (end 168.1099 135.0391) (width 0.45) (layer B.Cu) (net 14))
 (segment (start 165.1 138.557) (end 169.8625 138.557) (width 0.45) (layer B.Cu) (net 4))
 (segment (start 173.101 117.729) (end 171.704 116.332) (width 0.45) (layer B.Cu) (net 4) (status 20))
 (segment (start 173.101 131.572) (end 173.101 117.729) (width 0.45) (layer B.Cu) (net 4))
 (segment (start 173.101 135.3185) (end 173.101 131.572) (width 0.45) (layer B.Cu) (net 4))
 (segment (start 169.8625 138.557) (end 173.101 135.3185) (width 0.45) (layer B.Cu) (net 4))
 (segment (start 164.067 99.295) (end 164.067 107.044) (width 0.45) (layer B.Cu) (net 4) (status 10))
 (segment (start 171.704 114.681) (end 171.704 116.332) (width 0.45) (layer B.Cu) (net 4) (status 20))
 (segment (start 164.067 107.044) (end 171.704 114.681) (width 0.45) (layer B.Cu) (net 4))
 (segment (start 165.1 141.097) (end 163.703 141.097) (width 0.45) (layer B.Cu) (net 13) (status 400000))
 (segment (start 161.8615 142.9385) (end 161.8615 146.3167) (width 0.45) (layer B.Cu) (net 13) (status 800000))
 (segment (start 163.703 141.097) (end 161.8615 142.9385) (width 0.45) (layer B.Cu) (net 13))
 (segment (start 165.1 141.097) (end 165.9636 141.097) (width 0.45) (layer B.Cu) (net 13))
 (segment (start 165.9636 141.097) (end 167.4495 142.5829) (width 0.45) (layer B.Cu) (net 13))
 (segment (start 157.5816 157.0736) (end 155.575 155.067) (width 0.45) (layer B.Cu) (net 13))
 (segment (start 162.56 157.0736) (end 157.5816 157.0736) (width 0.45) (layer B.Cu) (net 13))
 (segment (start 167.4495 152.1841) (end 162.56 157.0736) (width 0.45) (layer B.Cu) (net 13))
 (segment (start 167.4495 142.5829) (end 167.4495 152.1841) (width 0.45) (layer B.Cu) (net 13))
 (segment (start 171.330251 128.133035) (end 171.330251 127.119749) (width 0.45) (layer B.Cu) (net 1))
 (segment (start 171.196 89.154) (end 167.64 85.598) (width 0.45) (layer B.Cu) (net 1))
 (segment (start 171.196 93.091) (end 171.196 89.154) (width 0.45) (layer B.Cu) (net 1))
 (segment (start 172.466 94.361) (end 171.196 93.091) (width 0.45) (layer B.Cu) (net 1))
 (via (at 172.466 94.361) (size 1.4) (drill 1) (layers F.Cu B.Cu) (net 1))
 (segment (start 173.482 95.377) (end 172.466 94.361) (width 0.45) (layer F.Cu) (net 1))
 (segment (start 173.482 124.968) (end 173.482 95.377) (width 0.45) (layer F.Cu) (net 1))
 (segment (start 171.831 126.619) (end 173.482 124.968) (width 0.45) (layer F.Cu) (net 1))
 (via (at 171.831 126.619) (size 1.4) (drill 1) (layers F.Cu B.Cu) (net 1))
 (segment (start 171.330251 127.119749) (end 171.831 126.619) (width 0.45) (layer B.Cu) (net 1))
 (segment (start 160.02 151.257) (end 160.02 150.8252) (width 0.45) (layer B.Cu) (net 12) (status C00000))
 (segment (start 160.02 150.8252) (end 158.6484 149.4536) (width 0.45) (layer B.Cu) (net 12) (status 400000))
 (segment (start 158.6484 149.4536) (end 157.2387 149.4536) (width 0.45) (layer B.Cu) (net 12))
 (segment (start 157.2387 149.4536) (end 152.3238 154.3685) (width 0.45) (layer B.Cu) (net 12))
 (segment (start 152.3238 154.3685) (end 147.2565 154.3685) (width 0.45) (layer B.Cu) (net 12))
 (segment (start 147.2565 154.3685) (end 146.05 153.162) (width 0.45) (layer B.Cu) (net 12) (status 800000))
 (segment (start 162.56 151.257) (end 162.56 150.9903) (width 0.45) (layer B.Cu) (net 11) (status C00000))
 (segment (start 162.56 150.9903) (end 159.9819 148.4122) (width 0.45) (layer B.Cu) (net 11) (status 400000))
 (segment (start 159.9819 148.4122) (end 155.8544 148.4122) (width 0.45) (layer B.Cu) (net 11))
 (segment (start 155.8544 148.4122) (end 151.2697 152.9969) (width 0.45) (layer B.Cu) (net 11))
 (segment (start 151.2697 152.9969) (end 148.4249 152.9969) (width 0.45) (layer B.Cu) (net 11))
 (segment (start 148.4249 152.9969) (end 146.05 150.622) (width 0.45) (layer B.Cu) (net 11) (status 800000))
 (segment (start 146.05 148.082) (end 146.685 148.082) (width 0.45) (layer B.Cu) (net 23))
 (segment (start 146.685 148.082) (end 149.86 151.257) (width 0.45) (layer B.Cu) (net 23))
 (segment (start 146.05 130.302) (end 146.6977 130.302) (width 0.45) (layer B.Cu) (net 16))
 (segment (start 146.6977 130.302) (end 149.86 133.4643) (width 0.45) (layer B.Cu) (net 16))
 (segment (start 149.86 133.4643) (end 149.86 133.477) (width 0.45) (layer B.Cu) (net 16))
 (segment (start 146.05 132.842) (end 146.685 132.842) (width 0.45) (layer B.Cu) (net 17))
 (segment (start 146.685 132.842) (end 149.86 136.017) (width 0.45) (layer B.Cu) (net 17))
 (segment (start 146.05 135.382) (end 146.685 135.382) (width 0.45) (layer B.Cu) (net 18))
 (segment (start 146.685 135.382) (end 149.86 138.557) (width 0.45) (layer B.Cu) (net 18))
 (segment (start 146.05 137.922) (end 146.685 137.922) (width 0.45) (layer B.Cu) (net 19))
 (segment (start 146.685 137.922) (end 149.86 141.097) (width 0.45) (layer B.Cu) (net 19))
 (segment (start 146.05 140.462) (end 146.685 140.462) (width 0.45) (layer B.Cu) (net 20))
 (segment (start 146.685 140.462) (end 149.86 143.637) (width 0.45) (layer B.Cu) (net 20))
 (segment (start 146.05 143.002) (end 146.685 143.002) (width 0.45) (layer B.Cu) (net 21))
 (segment (start 146.685 143.002) (end 149.86 146.177) (width 0.45) (layer B.Cu) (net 21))
 (segment (start 146.05 145.542) (end 146.685 145.542) (width 0.45) (layer B.Cu) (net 22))
 (segment (start 146.685 145.542) (end 149.86 148.717) (width 0.45) (layer B.Cu) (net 22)))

